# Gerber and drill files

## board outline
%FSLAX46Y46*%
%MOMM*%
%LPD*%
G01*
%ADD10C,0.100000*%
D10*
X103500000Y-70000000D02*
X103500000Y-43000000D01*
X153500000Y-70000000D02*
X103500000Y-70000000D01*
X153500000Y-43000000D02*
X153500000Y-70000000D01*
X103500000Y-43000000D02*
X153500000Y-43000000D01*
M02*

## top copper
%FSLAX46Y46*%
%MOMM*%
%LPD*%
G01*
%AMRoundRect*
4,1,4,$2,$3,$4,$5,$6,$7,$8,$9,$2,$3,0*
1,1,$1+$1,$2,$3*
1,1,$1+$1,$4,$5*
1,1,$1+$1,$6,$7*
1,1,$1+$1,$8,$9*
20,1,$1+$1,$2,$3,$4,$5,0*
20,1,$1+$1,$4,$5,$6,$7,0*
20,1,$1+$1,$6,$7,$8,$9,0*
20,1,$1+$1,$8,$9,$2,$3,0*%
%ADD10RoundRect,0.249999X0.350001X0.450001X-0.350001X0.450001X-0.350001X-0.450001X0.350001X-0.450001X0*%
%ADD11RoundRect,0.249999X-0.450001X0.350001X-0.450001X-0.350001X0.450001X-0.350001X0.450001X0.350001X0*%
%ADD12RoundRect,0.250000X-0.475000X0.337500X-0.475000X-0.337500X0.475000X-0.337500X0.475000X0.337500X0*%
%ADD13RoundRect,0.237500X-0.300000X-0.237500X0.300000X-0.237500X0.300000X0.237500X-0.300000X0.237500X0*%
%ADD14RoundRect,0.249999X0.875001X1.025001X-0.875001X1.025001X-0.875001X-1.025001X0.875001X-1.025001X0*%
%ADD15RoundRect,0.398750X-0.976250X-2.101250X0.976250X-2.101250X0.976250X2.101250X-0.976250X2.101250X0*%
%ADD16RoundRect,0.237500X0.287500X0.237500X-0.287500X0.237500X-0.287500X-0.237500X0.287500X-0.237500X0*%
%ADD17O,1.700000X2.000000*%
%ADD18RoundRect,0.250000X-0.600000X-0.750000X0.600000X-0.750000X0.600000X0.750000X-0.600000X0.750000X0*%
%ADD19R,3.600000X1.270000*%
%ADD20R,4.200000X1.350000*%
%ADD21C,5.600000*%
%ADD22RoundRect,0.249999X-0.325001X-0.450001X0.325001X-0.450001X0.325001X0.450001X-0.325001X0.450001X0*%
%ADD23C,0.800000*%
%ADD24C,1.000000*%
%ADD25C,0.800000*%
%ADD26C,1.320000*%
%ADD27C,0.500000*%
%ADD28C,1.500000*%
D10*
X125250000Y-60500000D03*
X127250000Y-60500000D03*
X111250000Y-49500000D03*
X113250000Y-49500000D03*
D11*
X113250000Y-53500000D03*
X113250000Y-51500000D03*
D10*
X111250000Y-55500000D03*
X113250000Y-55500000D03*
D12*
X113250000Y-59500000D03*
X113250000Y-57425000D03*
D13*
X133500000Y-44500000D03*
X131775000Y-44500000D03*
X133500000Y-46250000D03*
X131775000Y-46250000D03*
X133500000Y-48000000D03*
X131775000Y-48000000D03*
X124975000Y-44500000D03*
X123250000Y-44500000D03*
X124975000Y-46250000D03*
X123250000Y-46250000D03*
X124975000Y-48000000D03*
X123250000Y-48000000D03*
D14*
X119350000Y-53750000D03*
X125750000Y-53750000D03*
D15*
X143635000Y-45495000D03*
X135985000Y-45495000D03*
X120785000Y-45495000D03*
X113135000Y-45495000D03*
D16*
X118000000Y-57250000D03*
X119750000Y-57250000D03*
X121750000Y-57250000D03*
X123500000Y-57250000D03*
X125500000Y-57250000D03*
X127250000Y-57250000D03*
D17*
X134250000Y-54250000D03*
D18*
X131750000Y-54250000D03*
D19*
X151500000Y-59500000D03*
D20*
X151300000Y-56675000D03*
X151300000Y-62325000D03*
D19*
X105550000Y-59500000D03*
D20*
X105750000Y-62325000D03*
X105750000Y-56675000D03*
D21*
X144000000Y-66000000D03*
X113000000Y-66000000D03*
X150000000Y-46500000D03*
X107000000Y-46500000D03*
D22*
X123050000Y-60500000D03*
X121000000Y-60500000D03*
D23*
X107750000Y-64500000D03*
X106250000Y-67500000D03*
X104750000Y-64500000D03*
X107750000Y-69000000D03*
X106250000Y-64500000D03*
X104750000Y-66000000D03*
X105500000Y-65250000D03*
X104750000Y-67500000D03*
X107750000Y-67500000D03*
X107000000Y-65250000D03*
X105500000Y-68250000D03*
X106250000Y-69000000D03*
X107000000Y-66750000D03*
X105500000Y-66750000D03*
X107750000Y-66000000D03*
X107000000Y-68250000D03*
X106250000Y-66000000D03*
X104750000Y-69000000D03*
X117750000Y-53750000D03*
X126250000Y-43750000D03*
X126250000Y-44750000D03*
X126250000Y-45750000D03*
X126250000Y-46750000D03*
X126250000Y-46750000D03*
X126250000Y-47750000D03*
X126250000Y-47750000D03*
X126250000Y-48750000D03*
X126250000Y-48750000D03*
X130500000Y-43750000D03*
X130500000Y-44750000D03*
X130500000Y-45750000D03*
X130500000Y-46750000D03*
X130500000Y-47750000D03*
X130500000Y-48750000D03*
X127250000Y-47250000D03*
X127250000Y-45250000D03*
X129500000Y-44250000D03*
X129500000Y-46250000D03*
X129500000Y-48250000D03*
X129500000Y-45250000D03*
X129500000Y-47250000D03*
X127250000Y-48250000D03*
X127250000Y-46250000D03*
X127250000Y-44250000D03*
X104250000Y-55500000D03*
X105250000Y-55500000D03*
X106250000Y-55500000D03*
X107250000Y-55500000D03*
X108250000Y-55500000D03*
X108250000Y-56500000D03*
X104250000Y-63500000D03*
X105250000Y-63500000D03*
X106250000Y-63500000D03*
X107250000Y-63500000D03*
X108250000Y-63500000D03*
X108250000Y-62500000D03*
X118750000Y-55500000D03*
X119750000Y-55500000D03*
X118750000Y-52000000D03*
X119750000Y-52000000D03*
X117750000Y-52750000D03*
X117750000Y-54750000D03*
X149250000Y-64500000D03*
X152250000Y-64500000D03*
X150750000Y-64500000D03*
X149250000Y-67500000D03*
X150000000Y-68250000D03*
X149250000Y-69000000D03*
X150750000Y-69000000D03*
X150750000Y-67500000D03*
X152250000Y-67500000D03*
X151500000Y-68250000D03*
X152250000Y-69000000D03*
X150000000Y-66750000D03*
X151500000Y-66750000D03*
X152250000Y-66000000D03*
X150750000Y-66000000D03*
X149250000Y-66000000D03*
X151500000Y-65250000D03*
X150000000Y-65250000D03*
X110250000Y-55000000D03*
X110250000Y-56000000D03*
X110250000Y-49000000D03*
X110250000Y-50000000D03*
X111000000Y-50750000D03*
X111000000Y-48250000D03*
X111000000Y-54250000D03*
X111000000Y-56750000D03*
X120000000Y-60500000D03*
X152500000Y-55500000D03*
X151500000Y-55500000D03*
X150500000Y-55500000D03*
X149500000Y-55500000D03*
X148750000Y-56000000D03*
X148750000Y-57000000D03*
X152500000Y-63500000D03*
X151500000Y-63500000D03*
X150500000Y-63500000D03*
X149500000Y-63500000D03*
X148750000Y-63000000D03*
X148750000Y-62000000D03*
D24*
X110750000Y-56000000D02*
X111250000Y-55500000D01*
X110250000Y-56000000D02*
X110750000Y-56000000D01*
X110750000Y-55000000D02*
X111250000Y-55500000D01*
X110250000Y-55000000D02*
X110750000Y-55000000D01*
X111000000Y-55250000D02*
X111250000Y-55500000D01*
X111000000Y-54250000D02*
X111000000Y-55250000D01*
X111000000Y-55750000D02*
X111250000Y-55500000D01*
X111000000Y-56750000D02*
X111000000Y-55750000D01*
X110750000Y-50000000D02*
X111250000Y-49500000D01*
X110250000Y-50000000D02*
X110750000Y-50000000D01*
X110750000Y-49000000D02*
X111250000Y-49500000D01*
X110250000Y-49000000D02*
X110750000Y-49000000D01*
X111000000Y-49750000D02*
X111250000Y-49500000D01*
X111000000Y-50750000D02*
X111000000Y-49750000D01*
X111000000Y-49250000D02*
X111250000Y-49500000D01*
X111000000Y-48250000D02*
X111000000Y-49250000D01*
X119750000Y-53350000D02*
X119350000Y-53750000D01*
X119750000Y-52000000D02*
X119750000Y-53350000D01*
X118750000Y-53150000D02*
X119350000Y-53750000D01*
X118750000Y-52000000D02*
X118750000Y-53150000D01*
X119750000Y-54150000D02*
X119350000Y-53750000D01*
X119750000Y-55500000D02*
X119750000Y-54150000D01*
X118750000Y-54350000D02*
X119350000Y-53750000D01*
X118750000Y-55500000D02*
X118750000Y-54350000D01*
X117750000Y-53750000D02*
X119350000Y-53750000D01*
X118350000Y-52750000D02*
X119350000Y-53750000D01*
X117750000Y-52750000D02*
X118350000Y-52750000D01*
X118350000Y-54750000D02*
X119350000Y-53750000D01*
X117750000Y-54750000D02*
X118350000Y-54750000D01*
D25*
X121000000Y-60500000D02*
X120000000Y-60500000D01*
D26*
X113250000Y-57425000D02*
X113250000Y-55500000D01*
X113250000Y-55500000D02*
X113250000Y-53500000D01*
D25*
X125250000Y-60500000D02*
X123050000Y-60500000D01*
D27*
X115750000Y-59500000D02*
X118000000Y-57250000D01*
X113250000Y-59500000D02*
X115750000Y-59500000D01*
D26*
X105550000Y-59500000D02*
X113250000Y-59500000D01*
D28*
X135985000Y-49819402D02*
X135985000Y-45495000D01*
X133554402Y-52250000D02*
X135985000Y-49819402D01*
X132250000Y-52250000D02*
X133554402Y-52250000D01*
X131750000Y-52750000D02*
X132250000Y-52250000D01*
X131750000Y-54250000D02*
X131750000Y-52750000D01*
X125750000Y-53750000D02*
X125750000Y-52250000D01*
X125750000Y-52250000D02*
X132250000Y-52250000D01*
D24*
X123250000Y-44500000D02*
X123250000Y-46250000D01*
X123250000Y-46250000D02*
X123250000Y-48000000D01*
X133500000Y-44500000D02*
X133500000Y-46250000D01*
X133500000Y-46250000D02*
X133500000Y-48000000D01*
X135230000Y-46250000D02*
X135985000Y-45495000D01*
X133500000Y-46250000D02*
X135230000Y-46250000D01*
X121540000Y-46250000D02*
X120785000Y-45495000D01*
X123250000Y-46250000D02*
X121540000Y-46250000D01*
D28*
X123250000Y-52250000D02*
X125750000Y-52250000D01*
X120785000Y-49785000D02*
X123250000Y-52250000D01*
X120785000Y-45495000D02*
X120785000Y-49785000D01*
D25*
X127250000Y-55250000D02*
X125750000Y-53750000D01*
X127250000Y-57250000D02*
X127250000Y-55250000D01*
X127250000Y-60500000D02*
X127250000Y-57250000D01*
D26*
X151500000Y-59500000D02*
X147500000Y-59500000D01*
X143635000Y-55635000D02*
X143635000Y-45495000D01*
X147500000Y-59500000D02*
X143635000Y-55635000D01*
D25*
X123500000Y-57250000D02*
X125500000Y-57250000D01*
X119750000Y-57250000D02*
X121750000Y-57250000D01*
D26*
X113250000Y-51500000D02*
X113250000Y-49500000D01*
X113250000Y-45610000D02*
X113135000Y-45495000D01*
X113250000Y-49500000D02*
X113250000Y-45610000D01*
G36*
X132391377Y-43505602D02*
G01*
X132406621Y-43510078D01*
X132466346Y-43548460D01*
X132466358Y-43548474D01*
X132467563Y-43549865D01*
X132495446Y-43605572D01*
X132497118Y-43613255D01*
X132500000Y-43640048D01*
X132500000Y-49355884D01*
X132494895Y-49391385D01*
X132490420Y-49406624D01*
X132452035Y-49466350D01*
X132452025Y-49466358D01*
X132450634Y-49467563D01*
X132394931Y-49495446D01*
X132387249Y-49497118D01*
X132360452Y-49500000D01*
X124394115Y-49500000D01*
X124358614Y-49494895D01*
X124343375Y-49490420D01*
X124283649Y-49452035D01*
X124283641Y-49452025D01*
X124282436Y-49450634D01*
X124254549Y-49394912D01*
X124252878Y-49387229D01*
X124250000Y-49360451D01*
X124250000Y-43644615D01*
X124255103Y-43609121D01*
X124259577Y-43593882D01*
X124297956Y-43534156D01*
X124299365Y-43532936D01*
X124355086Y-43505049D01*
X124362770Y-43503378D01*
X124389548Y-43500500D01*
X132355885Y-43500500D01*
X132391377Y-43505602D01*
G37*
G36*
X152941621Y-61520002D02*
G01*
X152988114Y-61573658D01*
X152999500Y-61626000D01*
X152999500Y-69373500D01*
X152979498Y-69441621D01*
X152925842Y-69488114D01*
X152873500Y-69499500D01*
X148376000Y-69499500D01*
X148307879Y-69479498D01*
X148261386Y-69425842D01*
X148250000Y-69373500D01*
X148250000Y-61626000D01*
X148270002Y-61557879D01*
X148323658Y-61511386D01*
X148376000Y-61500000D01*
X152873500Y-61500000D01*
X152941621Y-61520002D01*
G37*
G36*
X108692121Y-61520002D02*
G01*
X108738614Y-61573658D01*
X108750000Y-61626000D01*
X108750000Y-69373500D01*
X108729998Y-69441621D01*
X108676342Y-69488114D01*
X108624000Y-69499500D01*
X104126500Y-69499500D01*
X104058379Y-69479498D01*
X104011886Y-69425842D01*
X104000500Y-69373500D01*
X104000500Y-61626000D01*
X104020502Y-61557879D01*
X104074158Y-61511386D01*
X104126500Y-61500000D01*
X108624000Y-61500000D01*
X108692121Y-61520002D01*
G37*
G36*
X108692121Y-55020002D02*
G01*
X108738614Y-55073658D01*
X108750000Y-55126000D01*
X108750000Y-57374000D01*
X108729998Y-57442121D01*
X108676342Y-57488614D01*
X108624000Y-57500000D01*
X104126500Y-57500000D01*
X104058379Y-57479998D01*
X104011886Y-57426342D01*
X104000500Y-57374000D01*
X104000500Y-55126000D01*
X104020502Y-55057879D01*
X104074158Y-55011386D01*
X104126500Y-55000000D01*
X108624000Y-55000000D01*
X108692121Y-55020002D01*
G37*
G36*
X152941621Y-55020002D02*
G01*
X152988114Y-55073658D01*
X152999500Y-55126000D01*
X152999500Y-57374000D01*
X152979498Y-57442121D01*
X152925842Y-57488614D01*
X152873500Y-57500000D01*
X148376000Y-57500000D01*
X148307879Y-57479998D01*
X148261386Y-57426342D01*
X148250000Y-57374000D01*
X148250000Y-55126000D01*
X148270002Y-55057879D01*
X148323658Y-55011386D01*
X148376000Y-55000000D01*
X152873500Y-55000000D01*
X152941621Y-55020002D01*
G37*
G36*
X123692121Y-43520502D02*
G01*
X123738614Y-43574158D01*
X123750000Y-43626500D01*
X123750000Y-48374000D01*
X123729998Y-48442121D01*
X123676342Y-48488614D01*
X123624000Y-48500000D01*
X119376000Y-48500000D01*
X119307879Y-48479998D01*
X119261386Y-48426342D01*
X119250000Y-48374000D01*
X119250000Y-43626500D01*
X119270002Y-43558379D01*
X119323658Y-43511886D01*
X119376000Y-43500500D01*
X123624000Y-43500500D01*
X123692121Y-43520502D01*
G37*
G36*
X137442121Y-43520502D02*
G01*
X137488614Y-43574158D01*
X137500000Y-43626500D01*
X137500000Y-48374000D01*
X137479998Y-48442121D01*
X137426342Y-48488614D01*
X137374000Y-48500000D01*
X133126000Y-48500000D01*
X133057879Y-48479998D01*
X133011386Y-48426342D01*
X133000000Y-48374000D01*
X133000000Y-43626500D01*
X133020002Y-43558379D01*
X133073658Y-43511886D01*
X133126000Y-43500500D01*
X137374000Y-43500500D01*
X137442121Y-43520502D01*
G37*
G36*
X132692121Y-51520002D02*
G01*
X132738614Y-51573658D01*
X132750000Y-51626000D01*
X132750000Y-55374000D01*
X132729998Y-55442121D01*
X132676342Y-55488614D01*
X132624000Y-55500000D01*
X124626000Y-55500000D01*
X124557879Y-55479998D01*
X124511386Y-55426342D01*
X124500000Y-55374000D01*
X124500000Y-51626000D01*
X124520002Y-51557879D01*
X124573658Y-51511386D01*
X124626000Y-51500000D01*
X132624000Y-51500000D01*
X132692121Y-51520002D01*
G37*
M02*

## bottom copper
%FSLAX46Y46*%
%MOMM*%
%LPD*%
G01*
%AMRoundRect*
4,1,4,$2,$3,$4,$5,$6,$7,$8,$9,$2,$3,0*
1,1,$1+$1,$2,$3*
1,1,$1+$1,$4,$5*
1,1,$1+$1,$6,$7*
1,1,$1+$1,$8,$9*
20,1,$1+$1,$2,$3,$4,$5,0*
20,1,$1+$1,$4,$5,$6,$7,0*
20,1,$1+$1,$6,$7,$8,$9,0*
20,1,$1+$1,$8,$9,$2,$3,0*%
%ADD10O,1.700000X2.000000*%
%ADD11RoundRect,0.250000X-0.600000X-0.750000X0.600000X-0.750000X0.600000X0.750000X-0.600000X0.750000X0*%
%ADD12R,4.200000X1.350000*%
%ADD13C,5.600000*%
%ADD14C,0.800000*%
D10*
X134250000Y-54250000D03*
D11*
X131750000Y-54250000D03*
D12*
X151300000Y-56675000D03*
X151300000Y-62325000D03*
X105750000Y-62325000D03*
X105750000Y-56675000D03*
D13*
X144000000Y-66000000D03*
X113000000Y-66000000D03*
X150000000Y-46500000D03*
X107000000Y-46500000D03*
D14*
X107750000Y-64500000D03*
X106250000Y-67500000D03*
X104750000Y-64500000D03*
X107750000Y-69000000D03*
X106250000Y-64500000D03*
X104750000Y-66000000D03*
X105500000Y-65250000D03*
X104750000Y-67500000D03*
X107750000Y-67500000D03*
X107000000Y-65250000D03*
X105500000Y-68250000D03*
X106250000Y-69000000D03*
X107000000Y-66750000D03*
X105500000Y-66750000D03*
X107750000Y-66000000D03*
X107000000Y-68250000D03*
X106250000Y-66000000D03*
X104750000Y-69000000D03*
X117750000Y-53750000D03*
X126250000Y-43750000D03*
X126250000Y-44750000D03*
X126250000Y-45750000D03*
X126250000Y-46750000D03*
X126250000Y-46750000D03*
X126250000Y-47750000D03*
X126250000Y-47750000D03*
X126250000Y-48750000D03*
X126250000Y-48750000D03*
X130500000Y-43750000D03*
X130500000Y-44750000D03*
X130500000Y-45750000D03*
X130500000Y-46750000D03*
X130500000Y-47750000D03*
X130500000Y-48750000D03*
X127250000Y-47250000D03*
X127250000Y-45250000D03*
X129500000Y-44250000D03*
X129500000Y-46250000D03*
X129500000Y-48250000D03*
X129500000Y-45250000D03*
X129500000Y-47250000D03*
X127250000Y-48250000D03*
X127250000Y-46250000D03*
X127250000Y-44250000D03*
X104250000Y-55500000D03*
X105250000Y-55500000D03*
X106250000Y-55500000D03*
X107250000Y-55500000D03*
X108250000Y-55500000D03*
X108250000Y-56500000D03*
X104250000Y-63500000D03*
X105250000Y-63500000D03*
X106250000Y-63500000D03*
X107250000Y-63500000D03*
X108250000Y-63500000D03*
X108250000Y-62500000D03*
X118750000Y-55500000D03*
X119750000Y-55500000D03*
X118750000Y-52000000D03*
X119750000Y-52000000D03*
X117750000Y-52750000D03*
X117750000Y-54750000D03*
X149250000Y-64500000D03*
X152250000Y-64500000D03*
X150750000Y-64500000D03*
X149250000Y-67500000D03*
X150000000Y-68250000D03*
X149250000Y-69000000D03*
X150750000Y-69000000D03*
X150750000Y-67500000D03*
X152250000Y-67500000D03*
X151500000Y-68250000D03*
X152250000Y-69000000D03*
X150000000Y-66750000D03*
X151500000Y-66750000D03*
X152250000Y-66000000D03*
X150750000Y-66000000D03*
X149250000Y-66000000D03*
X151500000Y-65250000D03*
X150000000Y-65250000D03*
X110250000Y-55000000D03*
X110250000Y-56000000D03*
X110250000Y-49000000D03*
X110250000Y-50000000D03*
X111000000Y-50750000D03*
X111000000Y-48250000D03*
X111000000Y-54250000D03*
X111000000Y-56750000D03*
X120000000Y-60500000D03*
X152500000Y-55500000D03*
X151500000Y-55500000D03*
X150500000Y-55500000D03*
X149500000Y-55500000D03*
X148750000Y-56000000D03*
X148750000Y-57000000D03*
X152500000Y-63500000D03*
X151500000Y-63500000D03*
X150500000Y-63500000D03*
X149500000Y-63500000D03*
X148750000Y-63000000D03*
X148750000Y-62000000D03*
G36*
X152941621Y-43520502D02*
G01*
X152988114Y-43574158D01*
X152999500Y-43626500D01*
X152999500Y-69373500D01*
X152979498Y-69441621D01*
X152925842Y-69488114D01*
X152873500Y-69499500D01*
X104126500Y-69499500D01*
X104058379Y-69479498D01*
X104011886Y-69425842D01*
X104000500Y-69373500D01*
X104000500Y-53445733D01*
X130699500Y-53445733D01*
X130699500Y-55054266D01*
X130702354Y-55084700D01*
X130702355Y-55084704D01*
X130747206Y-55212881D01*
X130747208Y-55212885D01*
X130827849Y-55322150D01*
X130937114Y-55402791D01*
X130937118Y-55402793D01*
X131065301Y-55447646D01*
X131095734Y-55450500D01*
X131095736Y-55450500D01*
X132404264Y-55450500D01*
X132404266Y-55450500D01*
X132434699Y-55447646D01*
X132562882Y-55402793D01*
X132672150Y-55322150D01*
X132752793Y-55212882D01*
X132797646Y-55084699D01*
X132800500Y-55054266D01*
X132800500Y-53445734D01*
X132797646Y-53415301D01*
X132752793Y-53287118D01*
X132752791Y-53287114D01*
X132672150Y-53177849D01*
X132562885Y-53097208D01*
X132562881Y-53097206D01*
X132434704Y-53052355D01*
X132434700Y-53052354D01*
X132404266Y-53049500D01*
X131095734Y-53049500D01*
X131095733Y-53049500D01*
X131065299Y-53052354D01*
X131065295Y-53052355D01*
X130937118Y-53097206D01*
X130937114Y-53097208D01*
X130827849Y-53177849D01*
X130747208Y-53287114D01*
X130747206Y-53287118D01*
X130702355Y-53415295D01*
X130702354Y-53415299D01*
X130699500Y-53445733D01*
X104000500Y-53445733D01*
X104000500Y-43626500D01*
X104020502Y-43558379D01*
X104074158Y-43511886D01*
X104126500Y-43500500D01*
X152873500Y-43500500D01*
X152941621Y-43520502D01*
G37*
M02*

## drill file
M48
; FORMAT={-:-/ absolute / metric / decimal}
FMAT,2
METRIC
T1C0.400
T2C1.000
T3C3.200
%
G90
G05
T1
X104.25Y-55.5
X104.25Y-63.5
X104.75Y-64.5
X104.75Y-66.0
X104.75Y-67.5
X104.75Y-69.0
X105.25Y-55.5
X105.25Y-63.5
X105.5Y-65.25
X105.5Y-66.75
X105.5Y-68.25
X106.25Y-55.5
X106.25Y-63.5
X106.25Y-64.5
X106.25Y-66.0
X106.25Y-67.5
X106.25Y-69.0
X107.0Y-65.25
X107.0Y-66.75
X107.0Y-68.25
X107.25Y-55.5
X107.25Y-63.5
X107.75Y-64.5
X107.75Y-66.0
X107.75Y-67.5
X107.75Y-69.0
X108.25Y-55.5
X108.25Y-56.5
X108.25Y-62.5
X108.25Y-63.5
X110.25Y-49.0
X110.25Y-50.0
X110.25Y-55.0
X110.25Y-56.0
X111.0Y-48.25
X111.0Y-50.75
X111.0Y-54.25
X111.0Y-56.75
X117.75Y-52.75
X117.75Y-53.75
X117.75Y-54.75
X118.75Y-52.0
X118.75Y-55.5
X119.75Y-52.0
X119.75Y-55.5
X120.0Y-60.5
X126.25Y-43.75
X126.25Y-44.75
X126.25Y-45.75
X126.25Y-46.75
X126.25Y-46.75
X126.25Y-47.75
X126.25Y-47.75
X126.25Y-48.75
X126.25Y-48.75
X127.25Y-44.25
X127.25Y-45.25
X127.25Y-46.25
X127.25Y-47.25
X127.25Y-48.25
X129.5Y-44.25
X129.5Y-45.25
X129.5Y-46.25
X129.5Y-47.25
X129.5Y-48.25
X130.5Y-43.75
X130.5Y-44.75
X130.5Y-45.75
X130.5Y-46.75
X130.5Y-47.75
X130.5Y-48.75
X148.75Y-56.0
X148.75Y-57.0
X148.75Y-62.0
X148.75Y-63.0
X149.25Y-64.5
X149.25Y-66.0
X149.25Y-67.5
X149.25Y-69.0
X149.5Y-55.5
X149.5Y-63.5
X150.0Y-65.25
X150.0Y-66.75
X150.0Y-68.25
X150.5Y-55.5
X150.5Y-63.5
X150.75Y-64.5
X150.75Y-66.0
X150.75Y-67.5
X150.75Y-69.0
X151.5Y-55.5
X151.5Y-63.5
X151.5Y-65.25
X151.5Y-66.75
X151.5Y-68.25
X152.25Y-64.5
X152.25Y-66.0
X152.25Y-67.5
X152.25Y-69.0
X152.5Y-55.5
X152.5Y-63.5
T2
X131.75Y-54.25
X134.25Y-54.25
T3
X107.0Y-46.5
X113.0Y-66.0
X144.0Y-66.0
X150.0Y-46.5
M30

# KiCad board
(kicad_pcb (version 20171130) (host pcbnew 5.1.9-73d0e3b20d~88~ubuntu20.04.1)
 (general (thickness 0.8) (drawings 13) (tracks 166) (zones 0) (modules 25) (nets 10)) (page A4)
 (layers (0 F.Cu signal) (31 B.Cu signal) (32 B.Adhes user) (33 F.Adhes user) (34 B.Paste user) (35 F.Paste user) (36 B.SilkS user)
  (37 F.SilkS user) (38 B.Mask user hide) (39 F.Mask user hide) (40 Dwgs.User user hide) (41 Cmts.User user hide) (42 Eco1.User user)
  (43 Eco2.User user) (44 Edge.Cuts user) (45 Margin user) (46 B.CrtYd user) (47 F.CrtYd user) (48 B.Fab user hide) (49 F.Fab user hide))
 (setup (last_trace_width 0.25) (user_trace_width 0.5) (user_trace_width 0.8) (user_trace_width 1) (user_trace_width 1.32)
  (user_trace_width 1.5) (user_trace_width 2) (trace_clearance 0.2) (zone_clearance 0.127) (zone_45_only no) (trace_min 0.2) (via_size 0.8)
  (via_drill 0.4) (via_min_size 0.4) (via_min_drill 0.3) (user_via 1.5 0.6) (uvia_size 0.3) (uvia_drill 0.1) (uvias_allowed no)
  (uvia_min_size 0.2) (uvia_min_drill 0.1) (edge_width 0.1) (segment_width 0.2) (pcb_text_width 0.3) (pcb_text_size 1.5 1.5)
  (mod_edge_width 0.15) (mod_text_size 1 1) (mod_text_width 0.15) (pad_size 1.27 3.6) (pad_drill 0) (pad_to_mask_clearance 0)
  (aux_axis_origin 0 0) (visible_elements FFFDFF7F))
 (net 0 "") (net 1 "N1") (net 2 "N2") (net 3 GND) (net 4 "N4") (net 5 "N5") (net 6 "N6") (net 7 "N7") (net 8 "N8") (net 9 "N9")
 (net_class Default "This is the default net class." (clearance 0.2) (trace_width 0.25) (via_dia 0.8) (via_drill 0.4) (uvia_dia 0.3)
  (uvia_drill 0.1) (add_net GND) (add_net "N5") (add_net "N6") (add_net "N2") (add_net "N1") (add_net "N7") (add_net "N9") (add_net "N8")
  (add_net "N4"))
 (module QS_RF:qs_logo (layer F.Cu) (at 122 67)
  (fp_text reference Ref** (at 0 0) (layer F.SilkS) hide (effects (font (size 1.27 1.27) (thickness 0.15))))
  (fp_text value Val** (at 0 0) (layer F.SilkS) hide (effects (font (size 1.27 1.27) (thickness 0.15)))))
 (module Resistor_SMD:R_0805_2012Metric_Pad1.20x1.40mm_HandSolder (layer F.Cu) (at 126.25 60.5 180)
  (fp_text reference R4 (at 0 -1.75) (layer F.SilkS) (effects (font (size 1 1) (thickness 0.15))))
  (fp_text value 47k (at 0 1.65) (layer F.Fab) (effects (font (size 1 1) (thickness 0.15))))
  (pad 2 smd roundrect (at 1 0 180) (size 1.2 1.4) (layers F.Cu F.Paste F.Mask) (roundrect_rratio 0.2083325) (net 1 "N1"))
  (pad 1 smd roundrect (at -1 0 180) (size 1.2 1.4) (layers F.Cu F.Paste F.Mask) (roundrect_rratio 0.2083325) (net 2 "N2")))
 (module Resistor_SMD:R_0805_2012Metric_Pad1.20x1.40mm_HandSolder (layer F.Cu) (at 112.25 49.5 180)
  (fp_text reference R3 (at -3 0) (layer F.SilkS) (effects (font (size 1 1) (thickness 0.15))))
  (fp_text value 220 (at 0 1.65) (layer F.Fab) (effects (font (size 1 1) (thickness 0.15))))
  (pad 2 smd roundrect (at 1 0 180) (size 1.2 1.4) (layers F.Cu F.Paste F.Mask) (roundrect_rratio 0.2083325) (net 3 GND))
  (pad 1 smd roundrect (at -1 0 180) (size 1.2 1.4) (layers F.Cu F.Paste F.Mask) (roundrect_rratio 0.2083325) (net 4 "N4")))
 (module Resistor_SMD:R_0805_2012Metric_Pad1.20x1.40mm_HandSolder (layer F.Cu) (at 113.25 52.5 270)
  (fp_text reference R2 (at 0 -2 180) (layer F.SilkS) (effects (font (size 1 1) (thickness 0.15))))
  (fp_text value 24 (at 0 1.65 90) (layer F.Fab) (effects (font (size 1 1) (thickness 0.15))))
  (pad 2 smd roundrect (at 1 0 270) (size 1.2 1.4) (layers F.Cu F.Paste F.Mask) (roundrect_rratio 0.2083325) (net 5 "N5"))
  (pad 1 smd roundrect (at -1 0 270) (size 1.2 1.4) (layers F.Cu F.Paste F.Mask) (roundrect_rratio 0.2083325) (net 4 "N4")))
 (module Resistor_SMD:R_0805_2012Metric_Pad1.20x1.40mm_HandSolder (layer F.Cu) (at 112.25 55.5 180)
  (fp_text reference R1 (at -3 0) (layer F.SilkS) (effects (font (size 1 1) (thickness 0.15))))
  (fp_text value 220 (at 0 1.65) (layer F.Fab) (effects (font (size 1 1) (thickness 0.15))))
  (pad 2 smd roundrect (at 1 0 180) (size 1.2 1.4) (layers F.Cu F.Paste F.Mask) (roundrect_rratio 0.2083325) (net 3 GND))
  (pad 1 smd roundrect (at -1 0 180) (size 1.2 1.4) (layers F.Cu F.Paste F.Mask) (roundrect_rratio 0.2083325) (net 5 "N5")))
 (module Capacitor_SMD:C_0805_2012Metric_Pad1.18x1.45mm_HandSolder (layer F.Cu) (at 113.25 58.4625 270)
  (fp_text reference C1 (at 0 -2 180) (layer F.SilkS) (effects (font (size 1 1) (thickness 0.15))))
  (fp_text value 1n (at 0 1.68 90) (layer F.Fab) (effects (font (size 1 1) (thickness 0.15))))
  (pad 2 smd roundrect (at 1.0375 0 270) (size 1.175 1.45) (layers F.Cu F.Paste F.Mask) (roundrect_rratio 0.2127659574468085) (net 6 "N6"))
  (pad 1 smd roundrect (at -1.0375 0 270) (size 1.175 1.45) (layers F.Cu F.Paste F.Mask) (roundrect_rratio 0.2127659574468085) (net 5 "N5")))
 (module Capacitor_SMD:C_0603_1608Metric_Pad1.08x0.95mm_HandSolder (layer F.Cu) (at 132.6375 44.5)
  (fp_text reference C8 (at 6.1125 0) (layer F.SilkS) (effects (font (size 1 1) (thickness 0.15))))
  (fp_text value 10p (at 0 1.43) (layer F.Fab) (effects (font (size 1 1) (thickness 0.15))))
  (pad 2 smd roundrect (at 0.8625 0) (size 1.075 0.95) (layers F.Cu F.Paste F.Mask) (roundrect_rratio 0.25) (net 2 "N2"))
  (pad 1 smd roundrect (at -0.8625 0) (size 1.075 0.95) (layers F.Cu F.Paste F.Mask) (roundrect_rratio 0.25) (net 3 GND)))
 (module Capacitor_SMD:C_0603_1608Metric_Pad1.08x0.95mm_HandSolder (layer F.Cu) (at 132.6375 46.25)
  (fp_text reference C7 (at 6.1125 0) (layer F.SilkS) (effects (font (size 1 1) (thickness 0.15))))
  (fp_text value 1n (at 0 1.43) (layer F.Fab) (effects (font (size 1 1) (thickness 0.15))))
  (pad 2 smd roundrect (at 0.8625 0) (size 1.075 0.95) (layers F.Cu F.Paste F.Mask) (roundrect_rratio 0.25) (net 2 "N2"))
  (pad 1 smd roundrect (at -0.8625 0) (size 1.075 0.95) (layers F.Cu F.Paste F.Mask) (roundrect_rratio 0.25) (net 3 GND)))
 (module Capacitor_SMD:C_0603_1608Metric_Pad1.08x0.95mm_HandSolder (layer F.Cu) (at 132.6375 48)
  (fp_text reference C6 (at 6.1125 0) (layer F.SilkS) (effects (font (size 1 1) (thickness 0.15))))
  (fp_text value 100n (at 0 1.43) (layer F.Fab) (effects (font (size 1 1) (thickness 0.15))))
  (pad 2 smd roundrect (at 0.8625 0) (size 1.075 0.95) (layers F.Cu F.Paste F.Mask) (roundrect_rratio 0.25) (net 2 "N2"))
  (pad 1 smd roundrect (at -0.8625 0) (size 1.075 0.95) (layers F.Cu F.Paste F.Mask) (roundrect_rratio 0.25) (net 3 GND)))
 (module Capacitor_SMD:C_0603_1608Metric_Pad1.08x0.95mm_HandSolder (layer F.Cu) (at 124.1125 44.5)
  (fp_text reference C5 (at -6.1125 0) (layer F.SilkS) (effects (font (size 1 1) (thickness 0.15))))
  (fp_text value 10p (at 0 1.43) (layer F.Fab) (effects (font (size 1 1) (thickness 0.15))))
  (pad 2 smd roundrect (at 0.8625 0) (size 1.075 0.95) (layers F.Cu F.Paste F.Mask) (roundrect_rratio 0.25) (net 3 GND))
  (pad 1 smd roundrect (at -0.8625 0) (size 1.075 0.95) (layers F.Cu F.Paste F.Mask) (roundrect_rratio 0.25) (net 2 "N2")))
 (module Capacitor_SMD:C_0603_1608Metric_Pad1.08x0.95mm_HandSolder (layer F.Cu) (at 124.1125 46.25)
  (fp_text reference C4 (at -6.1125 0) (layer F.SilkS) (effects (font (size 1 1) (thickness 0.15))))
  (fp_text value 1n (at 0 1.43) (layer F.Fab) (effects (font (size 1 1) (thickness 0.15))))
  (pad 2 smd roundrect (at 0.8625 0) (size 1.075 0.95) (layers F.Cu F.Paste F.Mask) (roundrect_rratio 0.25) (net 3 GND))
  (pad 1 smd roundrect (at -0.8625 0) (size 1.075 0.95) (layers F.Cu F.Paste F.Mask) (roundrect_rratio 0.25) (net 2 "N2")))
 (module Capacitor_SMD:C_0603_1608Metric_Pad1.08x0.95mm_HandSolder (layer F.Cu) (at 124.1125 48)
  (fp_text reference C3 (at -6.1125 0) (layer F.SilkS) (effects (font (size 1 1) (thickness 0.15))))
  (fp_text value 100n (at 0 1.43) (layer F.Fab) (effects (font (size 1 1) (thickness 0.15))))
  (pad 2 smd roundrect (at 0.8625 0) (size 1.075 0.95) (layers F.Cu F.Paste F.Mask) (roundrect_rratio 0.25) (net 3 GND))
  (pad 1 smd roundrect (at -0.8625 0) (size 1.075 0.95) (layers F.Cu F.Paste F.Mask) (roundrect_rratio 0.25) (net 2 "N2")))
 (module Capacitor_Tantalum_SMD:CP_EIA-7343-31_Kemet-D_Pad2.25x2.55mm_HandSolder (layer F.Cu) (at 122.55 53.75 180)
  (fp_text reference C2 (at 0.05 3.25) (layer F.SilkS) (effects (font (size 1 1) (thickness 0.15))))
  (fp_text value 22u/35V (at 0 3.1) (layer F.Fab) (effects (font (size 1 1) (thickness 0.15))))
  (pad 2 smd roundrect (at 3.2 0 180) (size 2.25 2.55) (layers F.Cu F.Paste F.Mask) (roundrect_rratio 0.1111106666666667) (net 3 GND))
  (pad 1 smd roundrect (at -3.2 0 180) (size 2.25 2.55) (layers F.Cu F.Paste F.Mask) (roundrect_rratio 0.1111106666666667) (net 2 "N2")))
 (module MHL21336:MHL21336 (layer F.Cu) (at 128.385 42.995)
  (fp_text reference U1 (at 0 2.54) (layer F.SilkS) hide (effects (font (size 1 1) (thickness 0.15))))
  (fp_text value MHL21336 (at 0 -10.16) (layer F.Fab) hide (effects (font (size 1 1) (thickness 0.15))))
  (pad 4 smd roundrect (at 15.25 2.5) (size 2.75 5) (layers F.Cu F.Paste F.Mask) (roundrect_rratio 0.145) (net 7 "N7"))
  (pad 3 smd roundrect (at 7.6 2.5) (size 2.75 5) (layers F.Cu F.Paste F.Mask) (roundrect_rratio 0.145) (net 2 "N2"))
  (pad 2 smd roundrect (at -7.6 2.5) (size 2.75 5) (layers F.Cu F.Paste F.Mask) (roundrect_rratio 0.145) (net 2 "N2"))
  (pad 1 smd roundrect (at -15.25 2.5) (size 2.75 5) (layers F.Cu F.Paste F.Mask) (roundrect_rratio 0.145) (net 4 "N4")))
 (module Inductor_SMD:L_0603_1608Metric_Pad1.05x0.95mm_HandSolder (layer F.Cu) (at 118.875 57.25 180)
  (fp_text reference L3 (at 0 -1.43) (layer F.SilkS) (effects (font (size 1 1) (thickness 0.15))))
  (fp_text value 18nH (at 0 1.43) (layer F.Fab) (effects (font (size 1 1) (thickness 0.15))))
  (pad 2 smd roundrect (at 0.875 0 180) (size 1.05 0.95) (layers F.Cu F.Paste F.Mask) (roundrect_rratio 0.25) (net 6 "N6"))
  (pad 1 smd roundrect (at -0.875 0 180) (size 1.05 0.95) (layers F.Cu F.Paste F.Mask) (roundrect_rratio 0.25) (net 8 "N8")))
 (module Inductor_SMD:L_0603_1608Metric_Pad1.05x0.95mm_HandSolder (layer F.Cu) (at 122.625 57.25 180)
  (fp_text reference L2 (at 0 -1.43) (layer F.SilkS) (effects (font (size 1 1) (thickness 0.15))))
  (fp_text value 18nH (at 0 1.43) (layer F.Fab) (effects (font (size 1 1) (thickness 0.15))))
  (pad 2 smd roundrect (at 0.875 0 180) (size 1.05 0.95) (layers F.Cu F.Paste F.Mask) (roundrect_rratio 0.25) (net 8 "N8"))
  (pad 1 smd roundrect (at -0.875 0 180) (size 1.05 0.95) (layers F.Cu F.Paste F.Mask) (roundrect_rratio 0.25) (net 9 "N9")))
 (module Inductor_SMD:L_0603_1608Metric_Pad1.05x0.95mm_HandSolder (layer F.Cu) (at 126.375 57.25 180)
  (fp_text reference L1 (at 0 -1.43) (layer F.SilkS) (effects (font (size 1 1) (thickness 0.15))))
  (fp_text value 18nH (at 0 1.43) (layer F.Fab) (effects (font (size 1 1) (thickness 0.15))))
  (pad 2 smd roundrect (at 0.875 0 180) (size 1.05 0.95) (layers F.Cu F.Paste F.Mask) (roundrect_rratio 0.25) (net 9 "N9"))
  (pad 1 smd roundrect (at -0.875 0 180) (size 1.05 0.95) (layers F.Cu F.Paste F.Mask) (roundrect_rratio 0.25) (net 2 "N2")))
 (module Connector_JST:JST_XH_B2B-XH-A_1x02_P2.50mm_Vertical (layer F.Cu) (at 131.75 54.25)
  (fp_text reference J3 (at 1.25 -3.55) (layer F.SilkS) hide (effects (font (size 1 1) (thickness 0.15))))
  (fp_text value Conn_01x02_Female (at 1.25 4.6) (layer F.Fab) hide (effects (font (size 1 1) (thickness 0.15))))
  (pad 2 thru_hole oval (at 2.5 0) (size 1.7 2) (drill 1) (layers *.Cu *.Mask) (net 3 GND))
  (pad 1 thru_hole roundrect (at 0 0) (size 1.7 2) (drill 1) (layers *.Cu *.Mask) (roundrect_rratio 0.1470588235294118) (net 2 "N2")))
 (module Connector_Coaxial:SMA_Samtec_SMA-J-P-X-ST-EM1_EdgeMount (layer F.Cu) (at 151.3 59.5 90)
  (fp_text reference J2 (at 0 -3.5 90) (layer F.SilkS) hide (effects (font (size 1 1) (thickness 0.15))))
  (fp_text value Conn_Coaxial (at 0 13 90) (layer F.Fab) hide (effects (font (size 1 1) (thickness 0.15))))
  (pad 1 smd rect (at 0 0.2 90) (size 1.27 3.6) (layers F.Cu F.Paste F.Mask) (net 7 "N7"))
  (pad 2 smd rect (at 2.825 0 90) (size 1.35 4.2) (layers F.Cu F.Paste F.Mask) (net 3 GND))
  (pad 2 smd rect (at -2.825 0 90) (size 1.35 4.2) (layers F.Cu F.Paste F.Mask) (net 3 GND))
  (pad 2 smd rect (at 2.825 0 90) (size 1.35 4.2) (layers B.Cu B.Paste B.Mask) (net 3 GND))
  (pad 2 smd rect (at -2.825 0 90) (size 1.35 4.2) (layers B.Cu B.Paste B.Mask) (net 3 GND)))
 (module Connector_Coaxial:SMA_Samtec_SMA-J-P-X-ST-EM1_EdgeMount (layer F.Cu) (at 105.75 59.5 270)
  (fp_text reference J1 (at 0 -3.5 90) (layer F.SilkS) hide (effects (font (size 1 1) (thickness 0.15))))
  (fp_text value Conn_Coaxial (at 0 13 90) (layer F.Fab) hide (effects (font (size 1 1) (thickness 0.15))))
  (pad 1 smd rect (at 0 0.2 270) (size 1.27 3.6) (layers F.Cu F.Paste F.Mask) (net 6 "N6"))
  (pad 2 smd rect (at 2.825 0 270) (size 1.35 4.2) (layers F.Cu F.Paste F.Mask) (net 3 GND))
  (pad 2 smd rect (at -2.825 0 270) (size 1.35 4.2) (layers F.Cu F.Paste F.Mask) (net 3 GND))
  (pad 2 smd rect (at 2.825 0 270) (size 1.35 4.2) (layers B.Cu B.Paste B.Mask) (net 3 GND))
  (pad 2 smd rect (at -2.825 0 270) (size 1.35 4.2) (layers B.Cu B.Paste B.Mask) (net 3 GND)))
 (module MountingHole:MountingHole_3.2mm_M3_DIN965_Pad (layer F.Cu) (at 144 66)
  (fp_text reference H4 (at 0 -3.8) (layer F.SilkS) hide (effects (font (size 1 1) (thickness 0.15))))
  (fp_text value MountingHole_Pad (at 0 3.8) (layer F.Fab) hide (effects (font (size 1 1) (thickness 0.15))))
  (pad 1 thru_hole circle (at 0 0) (size 5.6 5.6) (drill 3.2) (layers *.Cu *.Mask) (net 3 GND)))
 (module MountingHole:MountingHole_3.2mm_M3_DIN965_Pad (layer F.Cu) (at 113 66)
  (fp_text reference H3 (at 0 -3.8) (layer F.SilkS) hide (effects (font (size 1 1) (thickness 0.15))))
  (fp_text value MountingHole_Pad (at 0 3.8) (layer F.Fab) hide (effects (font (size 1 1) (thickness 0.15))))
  (pad 1 thru_hole circle (at 0 0) (size 5.6 5.6) (drill 3.2) (layers *.Cu *.Mask) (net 3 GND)))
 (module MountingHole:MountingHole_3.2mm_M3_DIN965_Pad (layer F.Cu) (at 150 46.5)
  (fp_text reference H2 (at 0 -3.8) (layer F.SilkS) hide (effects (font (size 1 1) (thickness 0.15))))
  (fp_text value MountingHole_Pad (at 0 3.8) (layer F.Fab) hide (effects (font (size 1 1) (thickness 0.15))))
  (pad 1 thru_hole circle (at 0 0) (size 5.6 5.6) (drill 3.2) (layers *.Cu *.Mask) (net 3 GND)))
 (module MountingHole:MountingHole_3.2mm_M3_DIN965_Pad (layer F.Cu) (at 107 46.5)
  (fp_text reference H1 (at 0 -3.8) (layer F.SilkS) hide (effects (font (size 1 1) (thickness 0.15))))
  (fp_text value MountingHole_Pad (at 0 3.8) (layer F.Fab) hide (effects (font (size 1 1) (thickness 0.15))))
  (pad 1 thru_hole circle (at 0 0) (size 5.6 5.6) (drill 3.2) (layers *.Cu *.Mask) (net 3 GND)))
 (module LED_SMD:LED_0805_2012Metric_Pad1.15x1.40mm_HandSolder (layer F.Cu) (at 122.025 60.5)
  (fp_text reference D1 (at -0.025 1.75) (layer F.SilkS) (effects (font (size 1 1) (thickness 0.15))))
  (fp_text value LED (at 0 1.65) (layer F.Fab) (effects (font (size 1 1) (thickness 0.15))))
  (pad 2 smd roundrect (at 1.025 0) (size 1.15 1.4) (layers F.Cu F.Paste F.Mask) (roundrect_rratio 0.2173904347826087) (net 1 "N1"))
  (pad 1 smd roundrect (at -1.025 0) (size 1.15 1.4) (layers F.Cu F.Paste F.Mask) (roundrect_rratio 0.2173904347826087) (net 3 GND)))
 (gr_line (start 103.5 70) (end 103.5 43) (layer Edge.Cuts) (width 0.1))
 (gr_line (start 153.5 70) (end 103.5 70) (layer Edge.Cuts) (width 0.1))
 (gr_line (start 153.5 43) (end 153.5 70) (layer Edge.Cuts) (width 0.1))
 (gr_line (start 103.5 43) (end 153.5 43) (layer Edge.Cuts) (width 0.1))
 (via (at 107.75 64.5) (size 0.8) (drill 0.4) (layers F.Cu B.Cu) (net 3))
 (via (at 106.25 67.5) (size 0.8) (drill 0.4) (layers F.Cu B.Cu) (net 3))
 (via (at 104.75 64.5) (size 0.8) (drill 0.4) (layers F.Cu B.Cu) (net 3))
 (via (at 107.75 69) (size 0.8) (drill 0.4) (layers F.Cu B.Cu) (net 3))
 (via (at 106.25 64.5) (size 0.8) (drill 0.4) (layers F.Cu B.Cu) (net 3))
 (via (at 104.75 66) (size 0.8) (drill 0.4) (layers F.Cu B.Cu) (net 3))
 (via (at 105.5 65.25) (size 0.8) (drill 0.4) (layers F.Cu B.Cu) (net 3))
 (via (at 104.75 67.5) (size 0.8) (drill 0.4) (layers F.Cu B.Cu) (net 3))
 (via (at 107.75 67.5) (size 0.8) (drill 0.4) (layers F.Cu B.Cu) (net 3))
 (via (at 107 65.25) (size 0.8) (drill 0.4) (layers F.Cu B.Cu) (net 3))
 (via (at 105.5 68.25) (size 0.8) (drill 0.4) (layers F.Cu B.Cu) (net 3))
 (via (at 106.25 69) (size 0.8) (drill 0.4) (layers F.Cu B.Cu) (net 3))
 (via (at 107 66.75) (size 0.8) (drill 0.4) (layers F.Cu B.Cu) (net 3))
 (via (at 105.5 66.75) (size 0.8) (drill 0.4) (layers F.Cu B.Cu) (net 3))
 (via (at 107.75 66) (size 0.8) (drill 0.4) (layers F.Cu B.Cu) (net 3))
 (via (at 107 68.25) (size 0.8) (drill 0.4) (layers F.Cu B.Cu) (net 3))
 (via (at 106.25 66) (size 0.8) (drill 0.4) (layers F.Cu B.Cu) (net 3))
 (via (at 104.75 69) (size 0.8) (drill 0.4) (layers F.Cu B.Cu) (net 3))
 (via (at 117.75 53.75) (size 0.8) (drill 0.4) (layers F.Cu B.Cu) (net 3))
 (via (at 126.25 43.75) (size 0.8) (drill 0.4) (layers F.Cu B.Cu) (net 3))
 (via (at 126.25 44.75) (size 0.8) (drill 0.4) (layers F.Cu B.Cu) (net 3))
 (via (at 126.25 45.75) (size 0.8) (drill 0.4) (layers F.Cu B.Cu) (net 3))
 (via (at 126.25 46.75) (size 0.8) (drill 0.4) (layers F.Cu B.Cu) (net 3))
 (via (at 126.25 46.75) (size 0.8) (drill 0.4) (layers F.Cu B.Cu) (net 3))
 (via (at 126.25 47.75) (size 0.8) (drill 0.4) (layers F.Cu B.Cu) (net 3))
 (via (at 126.25 47.75) (size 0.8) (drill 0.4) (layers F.Cu B.Cu) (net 3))
 (via (at 126.25 48.75) (size 0.8) (drill 0.4) (layers F.Cu B.Cu) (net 3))
 (via (at 126.25 48.75) (size 0.8) (drill 0.4) (layers F.Cu B.Cu) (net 3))
 (via (at 130.5 43.75) (size 0.8) (drill 0.4) (layers F.Cu B.Cu) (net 3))
 (via (at 130.5 44.75) (size 0.8) (drill 0.4) (layers F.Cu B.Cu) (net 3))
 (via (at 130.5 45.75) (size 0.8) (drill 0.4) (layers F.Cu B.Cu) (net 3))
 (via (at 130.5 46.75) (size 0.8) (drill 0.4) (layers F.Cu B.Cu) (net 3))
 (via (at 130.5 47.75) (size 0.8) (drill 0.4) (layers F.Cu B.Cu) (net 3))
 (via (at 130.5 48.75) (size 0.8) (drill 0.4) (layers F.Cu B.Cu) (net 3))
 (via (at 127.25 47.25) (size 0.8) (drill 0.4) (layers F.Cu B.Cu) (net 3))
 (via (at 127.25 45.25) (size 0.8) (drill 0.4) (layers F.Cu B.Cu) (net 3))
 (via (at 129.5 44.25) (size 0.8) (drill 0.4) (layers F.Cu B.Cu) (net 3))
 (via (at 129.5 46.25) (size 0.8) (drill 0.4) (layers F.Cu B.Cu) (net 3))
 (via (at 129.5 48.25) (size 0.8) (drill 0.4) (layers F.Cu B.Cu) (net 3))
 (via (at 129.5 45.25) (size 0.8) (drill 0.4) (layers F.Cu B.Cu) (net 3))
 (via (at 129.5 47.25) (size 0.8) (drill 0.4) (layers F.Cu B.Cu) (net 3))
 (via (at 127.25 48.25) (size 0.8) (drill 0.4) (layers F.Cu B.Cu) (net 3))
 (via (at 127.25 46.25) (size 0.8) (drill 0.4) (layers F.Cu B.Cu) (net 3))
 (via (at 127.25 44.25) (size 0.8) (drill 0.4) (layers F.Cu B.Cu) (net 3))
 (via (at 104.25 55.5) (size 0.8) (drill 0.4) (layers F.Cu B.Cu) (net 3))
 (via (at 105.25 55.5) (size 0.8) (drill 0.4) (layers F.Cu B.Cu) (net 3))
 (via (at 106.25 55.5) (size 0.8) (drill 0.4) (layers F.Cu B.Cu) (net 3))
 (via (at 107.25 55.5) (size 0.8) (drill 0.4) (layers F.Cu B.Cu) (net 3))
 (via (at 108.25 55.5) (size 0.8) (drill 0.4) (layers F.Cu B.Cu) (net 3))
 (via (at 108.25 56.5) (size 0.8) (drill 0.4) (layers F.Cu B.Cu) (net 3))
 (via (at 104.25 63.5) (size 0.8) (drill 0.4) (layers F.Cu B.Cu) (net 3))
 (via (at 105.25 63.5) (size 0.8) (drill 0.4) (layers F.Cu B.Cu) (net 3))
 (via (at 106.25 63.5) (size 0.8) (drill 0.4) (layers F.Cu B.Cu) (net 3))
 (via (at 107.25 63.5) (size 0.8) (drill 0.4) (layers F.Cu B.Cu) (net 3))
 (via (at 108.25 63.5) (size 0.8) (drill 0.4) (layers F.Cu B.Cu) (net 3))
 (via (at 108.25 62.5) (size 0.8) (drill 0.4) (layers F.Cu B.Cu) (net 3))
 (via (at 118.75 55.5) (size 0.8) (drill 0.4) (layers F.Cu B.Cu) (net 3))
 (via (at 119.75 55.5) (size 0.8) (drill 0.4) (layers F.Cu B.Cu) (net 3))
 (via (at 118.75 52) (size 0.8) (drill 0.4) (layers F.Cu B.Cu) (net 3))
 (via (at 119.75 52) (size 0.8) (drill 0.4) (layers F.Cu B.Cu) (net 3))
 (via (at 117.75 52.75) (size 0.8) (drill 0.4) (layers F.Cu B.Cu) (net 3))
 (via (at 117.75 54.75) (size 0.8) (drill 0.4) (layers F.Cu B.Cu) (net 3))
 (via (at 149.25 64.5) (size 0.8) (drill 0.4) (layers F.Cu B.Cu) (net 3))
 (via (at 152.25 64.5) (size 0.8) (drill 0.4) (layers F.Cu B.Cu) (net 3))
 (via (at 150.75 64.5) (size 0.8) (drill 0.4) (layers F.Cu B.Cu) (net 3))
 (via (at 149.25 67.5) (size 0.8) (drill 0.4) (layers F.Cu B.Cu) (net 3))
 (via (at 150 68.25) (size 0.8) (drill 0.4) (layers F.Cu B.Cu) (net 3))
 (via (at 149.25 69) (size 0.8) (drill 0.4) (layers F.Cu B.Cu) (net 3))
 (via (at 150.75 69) (size 0.8) (drill 0.4) (layers F.Cu B.Cu) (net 3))
 (via (at 150.75 67.5) (size 0.8) (drill 0.4) (layers F.Cu B.Cu) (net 3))
 (via (at 152.25 67.5) (size 0.8) (drill 0.4) (layers F.Cu B.Cu) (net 3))
 (via (at 151.5 68.25) (size 0.8) (drill 0.4) (layers F.Cu B.Cu) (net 3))
 (via (at 152.25 69) (size 0.8) (drill 0.4) (layers F.Cu B.Cu) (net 3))
 (via (at 150 66.75) (size 0.8) (drill 0.4) (layers F.Cu B.Cu) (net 3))
 (via (at 151.5 66.75) (size 0.8) (drill 0.4) (layers F.Cu B.Cu) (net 3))
 (via (at 152.25 66) (size 0.8) (drill 0.4) (layers F.Cu B.Cu) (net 3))
 (via (at 150.75 66) (size 0.8) (drill 0.4) (layers F.Cu B.Cu) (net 3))
 (via (at 149.25 66) (size 0.8) (drill 0.4) (layers F.Cu B.Cu) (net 3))
 (via (at 151.5 65.25) (size 0.8) (drill 0.4) (layers F.Cu B.Cu) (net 3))
 (via (at 150 65.25) (size 0.8) (drill 0.4) (layers F.Cu B.Cu) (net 3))
 (via (at 110.25 55) (size 0.8) (drill 0.4) (layers F.Cu B.Cu) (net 3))
 (via (at 110.25 56) (size 0.8) (drill 0.4) (layers F.Cu B.Cu) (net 3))
 (via (at 110.25 49) (size 0.8) (drill 0.4) (layers F.Cu B.Cu) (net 3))
 (via (at 110.25 50) (size 0.8) (drill 0.4) (layers F.Cu B.Cu) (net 3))
 (via (at 111 50.75) (size 0.8) (drill 0.4) (layers F.Cu B.Cu) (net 3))
 (via (at 111 48.25) (size 0.8) (drill 0.4) (layers F.Cu B.Cu) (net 3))
 (via (at 111 54.25) (size 0.8) (drill 0.4) (layers F.Cu B.Cu) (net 3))
 (via (at 111 56.75) (size 0.8) (drill 0.4) (layers F.Cu B.Cu) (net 3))
 (segment (start 110.75 56) (end 111.25 55.5) (width 1) (layer F.Cu) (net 3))
 (segment (start 110.25 56) (end 110.75 56) (width 1) (layer F.Cu) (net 3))
 (segment (start 110.75 55) (end 111.25 55.5) (width 1) (layer F.Cu) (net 3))
 (segment (start 110.25 55) (end 110.75 55) (width 1) (layer F.Cu) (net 3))
 (segment (start 111 55.25) (end 111.25 55.5) (width 1) (layer F.Cu) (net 3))
 (segment (start 111 54.25) (end 111 55.25) (width 1) (layer F.Cu) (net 3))
 (segment (start 111 55.75) (end 111.25 55.5) (width 1) (layer F.Cu) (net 3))
 (segment (start 111 56.75) (end 111 55.75) (width 1) (layer F.Cu) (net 3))
 (segment (start 110.75 50) (end 111.25 49.5) (width 1) (layer F.Cu) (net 3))
 (segment (start 110.25 50) (end 110.75 50) (width 1) (layer F.Cu) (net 3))
 (segment (start 110.75 49) (end 111.25 49.5) (width 1) (layer F.Cu) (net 3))
 (segment (start 110.25 49) (end 110.75 49) (width 1) (layer F.Cu) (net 3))
 (segment (start 111 49.75) (end 111.25 49.5) (width 1) (layer F.Cu) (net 3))
 (segment (start 111 50.75) (end 111 49.75) (width 1) (layer F.Cu) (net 3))
 (segment (start 111 49.25) (end 111.25 49.5) (width 1) (layer F.Cu) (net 3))
 (segment (start 111 48.25) (end 111 49.25) (width 1) (layer F.Cu) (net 3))
 (segment (start 119.75 53.35) (end 119.35 53.75) (width 1) (layer F.Cu) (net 3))
 (segment (start 119.75 52) (end 119.75 53.35) (width 1) (layer F.Cu) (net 3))
 (segment (start 118.75 53.15) (end 119.35 53.75) (width 1) (layer F.Cu) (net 3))
 (segment (start 118.75 52) (end 118.75 53.15) (width 1) (layer F.Cu) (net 3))
 (segment (start 119.75 54.15) (end 119.35 53.75) (width 1) (layer F.Cu) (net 3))
 (segment (start 119.75 55.5) (end 119.75 54.15) (width 1) (layer F.Cu) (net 3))
 (segment (start 118.75 54.35) (end 119.35 53.75) (width 1) (layer F.Cu) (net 3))
 (segment (start 118.75 55.5) (end 118.75 54.35) (width 1) (layer F.Cu) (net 3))
 (segment (start 117.75 53.75) (end 119.35 53.75) (width 1) (layer F.Cu) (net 3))
 (segment (start 118.35 52.75) (end 119.35 53.75) (width 1) (layer F.Cu) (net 3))
 (segment (start 117.75 52.75) (end 118.35 52.75) (width 1) (layer F.Cu) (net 3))
 (segment (start 118.35 54.75) (end 119.35 53.75) (width 1) (layer F.Cu) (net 3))
 (segment (start 117.75 54.75) (end 118.35 54.75) (width 1) (layer F.Cu) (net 3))
 (via (at 120 60.5) (size 0.8) (drill 0.4) (layers F.Cu B.Cu) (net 3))
 (segment (start 121 60.5) (end 120 60.5) (width 0.8) (layer F.Cu) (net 3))
 (via (at 152.5 55.5) (size 0.8) (drill 0.4) (layers F.Cu B.Cu) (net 3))
 (via (at 151.5 55.5) (size 0.8) (drill 0.4) (layers F.Cu B.Cu) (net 3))
 (via (at 150.5 55.5) (size 0.8) (drill 0.4) (layers F.Cu B.Cu) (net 3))
 (via (at 149.5 55.5) (size 0.8) (drill 0.4) (layers F.Cu B.Cu) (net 3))
 (via (at 148.75 56) (size 0.8) (drill 0.4) (layers F.Cu B.Cu) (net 3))
 (via (at 148.75 57) (size 0.8) (drill 0.4) (layers F.Cu B.Cu) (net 3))
 (via (at 152.5 63.5) (size 0.8) (drill 0.4) (layers F.Cu B.Cu) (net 3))
 (via (at 151.5 63.5) (size 0.8) (drill 0.4) (layers F.Cu B.Cu) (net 3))
 (via (at 150.5 63.5) (size 0.8) (drill 0.4) (layers F.Cu B.Cu) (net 3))
 (via (at 149.5 63.5) (size 0.8) (drill 0.4) (layers F.Cu B.Cu) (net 3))
 (via (at 148.75 63) (size 0.8) (drill 0.4) (layers F.Cu B.Cu) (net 3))
 (via (at 148.75 62) (size 0.8) (drill 0.4) (layers F.Cu B.Cu) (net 3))
 (segment (start 113.25 57.425) (end 113.25 55.5) (width 1.32) (layer F.Cu) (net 5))
 (segment (start 113.25 55.5) (end 113.25 53.5) (width 1.32) (layer F.Cu) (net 5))
 (segment (start 125.25 60.5) (end 123.05 60.5) (width 0.8) (layer F.Cu) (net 1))
 (segment (start 115.75 59.5) (end 118 57.25) (width 0.5) (layer F.Cu) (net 6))
 (segment (start 113.25 59.5) (end 115.75 59.5) (width 0.5) (layer F.Cu) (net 6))
 (segment (start 105.55 59.5) (end 113.25 59.5) (width 1.32) (layer F.Cu) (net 6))
 (segment (start 135.985 49.819402) (end 135.985 45.495) (width 1.5) (layer F.Cu) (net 2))
 (segment (start 133.554402 52.25) (end 135.985 49.819402) (width 1.5) (layer F.Cu) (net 2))
 (segment (start 132.25 52.25) (end 133.554402 52.25) (width 1.5) (layer F.Cu) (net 2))
 (segment (start 131.75 52.75) (end 132.25 52.25) (width 1.5) (layer F.Cu) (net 2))
 (segment (start 131.75 54.25) (end 131.75 52.75) (width 1.5) (layer F.Cu) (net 2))
 (segment (start 125.75 53.75) (end 125.75 52.25) (width 1.5) (layer F.Cu) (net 2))
 (segment (start 125.75 52.25) (end 132.25 52.25) (width 1.5) (layer F.Cu) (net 2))
 (segment (start 123.25 44.5) (end 123.25 46.25) (width 1) (layer F.Cu) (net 2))
 (segment (start 123.25 46.25) (end 123.25 48) (width 1) (layer F.Cu) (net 2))
 (segment (start 133.5 44.5) (end 133.5 46.25) (width 1) (layer F.Cu) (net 2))
 (segment (start 133.5 46.25) (end 133.5 48) (width 1) (layer F.Cu) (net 2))
 (segment (start 135.23 46.25) (end 135.985 45.495) (width 1) (layer F.Cu) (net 2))
 (segment (start 133.5 46.25) (end 135.23 46.25) (width 1) (layer F.Cu) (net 2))
 (segment (start 121.54 46.25) (end 120.785 45.495) (width 1) (layer F.Cu) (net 2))
 (segment (start 123.25 46.25) (end 121.54 46.25) (width 1) (layer F.Cu) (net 2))
 (segment (start 123.25 52.25) (end 125.75 52.25) (width 1.5) (layer F.Cu) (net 2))
 (segment (start 120.785 49.785) (end 123.25 52.25) (width 1.5) (layer F.Cu) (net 2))
 (segment (start 120.785 45.495) (end 120.785 49.785) (width 1.5) (layer F.Cu) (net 2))
 (segment (start 127.25 55.25) (end 125.75 53.75) (width 0.8) (layer F.Cu) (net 2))
 (segment (start 127.25 57.25) (end 127.25 55.25) (width 0.8) (layer F.Cu) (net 2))
 (segment (start 127.25 60.5) (end 127.25 57.25) (width 0.8) (layer F.Cu) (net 2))
 (segment (start 151.5 59.5) (end 147.5 59.5) (width 1.32) (layer F.Cu) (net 7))
 (segment (start 143.635 55.635) (end 143.635 45.495) (width 1.32) (layer F.Cu) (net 7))
 (segment (start 147.5 59.5) (end 143.635 55.635) (width 1.32) (layer F.Cu) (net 7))
 (segment (start 123.5 57.25) (end 125.5 57.25) (width 0.8) (layer F.Cu) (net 9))
 (segment (start 119.75 57.25) (end 121.75 57.25) (width 0.8) (layer F.Cu) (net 8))
 (segment (start 113.25 51.5) (end 113.25 49.5) (width 1.32) (layer F.Cu) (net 4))
 (segment (start 113.25 45.61) (end 113.135 45.495) (width 1.32) (layer F.Cu) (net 4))
 (segment (start 113.25 49.5) (end 113.25 45.61) (width 1.32) (layer F.Cu) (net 4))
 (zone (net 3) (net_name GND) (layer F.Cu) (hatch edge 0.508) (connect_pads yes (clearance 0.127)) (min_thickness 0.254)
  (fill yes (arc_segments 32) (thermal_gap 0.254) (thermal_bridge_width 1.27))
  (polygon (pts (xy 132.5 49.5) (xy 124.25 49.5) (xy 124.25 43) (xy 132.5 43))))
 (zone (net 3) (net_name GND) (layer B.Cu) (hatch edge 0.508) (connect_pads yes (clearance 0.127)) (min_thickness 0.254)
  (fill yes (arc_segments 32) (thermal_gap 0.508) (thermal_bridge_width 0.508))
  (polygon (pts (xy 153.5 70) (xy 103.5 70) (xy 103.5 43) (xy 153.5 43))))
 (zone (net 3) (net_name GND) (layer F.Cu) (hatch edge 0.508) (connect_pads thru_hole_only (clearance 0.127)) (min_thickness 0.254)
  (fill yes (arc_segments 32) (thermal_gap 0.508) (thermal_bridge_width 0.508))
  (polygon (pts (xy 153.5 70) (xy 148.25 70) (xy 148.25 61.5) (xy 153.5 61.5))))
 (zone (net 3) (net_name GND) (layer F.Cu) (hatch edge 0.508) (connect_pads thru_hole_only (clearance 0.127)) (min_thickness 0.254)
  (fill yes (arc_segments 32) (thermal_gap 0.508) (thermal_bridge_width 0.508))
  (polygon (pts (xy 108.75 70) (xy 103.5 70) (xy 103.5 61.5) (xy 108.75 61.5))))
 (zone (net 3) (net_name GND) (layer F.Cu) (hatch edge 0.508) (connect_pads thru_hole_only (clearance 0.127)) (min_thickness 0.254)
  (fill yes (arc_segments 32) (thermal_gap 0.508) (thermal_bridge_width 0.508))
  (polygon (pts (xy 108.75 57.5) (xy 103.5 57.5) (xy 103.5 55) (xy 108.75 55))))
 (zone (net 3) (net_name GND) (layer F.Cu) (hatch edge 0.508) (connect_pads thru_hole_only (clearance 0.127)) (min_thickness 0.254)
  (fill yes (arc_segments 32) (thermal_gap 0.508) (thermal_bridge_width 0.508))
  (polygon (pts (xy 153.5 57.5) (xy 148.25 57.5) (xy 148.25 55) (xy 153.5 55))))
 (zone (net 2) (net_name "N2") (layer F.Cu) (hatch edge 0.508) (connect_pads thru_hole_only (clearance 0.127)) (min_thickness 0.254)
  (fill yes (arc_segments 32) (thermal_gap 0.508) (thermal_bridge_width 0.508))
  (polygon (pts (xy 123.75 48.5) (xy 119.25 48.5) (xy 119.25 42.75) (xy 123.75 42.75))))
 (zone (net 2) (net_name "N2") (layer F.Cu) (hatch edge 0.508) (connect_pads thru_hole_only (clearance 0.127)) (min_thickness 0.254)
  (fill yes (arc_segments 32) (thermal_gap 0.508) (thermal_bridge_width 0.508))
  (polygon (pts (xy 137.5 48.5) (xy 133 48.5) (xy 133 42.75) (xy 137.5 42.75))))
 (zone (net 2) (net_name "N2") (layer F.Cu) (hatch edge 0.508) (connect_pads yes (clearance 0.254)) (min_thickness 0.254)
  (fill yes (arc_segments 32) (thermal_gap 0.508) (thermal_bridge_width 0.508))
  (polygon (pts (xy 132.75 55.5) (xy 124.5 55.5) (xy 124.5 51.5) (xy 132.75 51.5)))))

